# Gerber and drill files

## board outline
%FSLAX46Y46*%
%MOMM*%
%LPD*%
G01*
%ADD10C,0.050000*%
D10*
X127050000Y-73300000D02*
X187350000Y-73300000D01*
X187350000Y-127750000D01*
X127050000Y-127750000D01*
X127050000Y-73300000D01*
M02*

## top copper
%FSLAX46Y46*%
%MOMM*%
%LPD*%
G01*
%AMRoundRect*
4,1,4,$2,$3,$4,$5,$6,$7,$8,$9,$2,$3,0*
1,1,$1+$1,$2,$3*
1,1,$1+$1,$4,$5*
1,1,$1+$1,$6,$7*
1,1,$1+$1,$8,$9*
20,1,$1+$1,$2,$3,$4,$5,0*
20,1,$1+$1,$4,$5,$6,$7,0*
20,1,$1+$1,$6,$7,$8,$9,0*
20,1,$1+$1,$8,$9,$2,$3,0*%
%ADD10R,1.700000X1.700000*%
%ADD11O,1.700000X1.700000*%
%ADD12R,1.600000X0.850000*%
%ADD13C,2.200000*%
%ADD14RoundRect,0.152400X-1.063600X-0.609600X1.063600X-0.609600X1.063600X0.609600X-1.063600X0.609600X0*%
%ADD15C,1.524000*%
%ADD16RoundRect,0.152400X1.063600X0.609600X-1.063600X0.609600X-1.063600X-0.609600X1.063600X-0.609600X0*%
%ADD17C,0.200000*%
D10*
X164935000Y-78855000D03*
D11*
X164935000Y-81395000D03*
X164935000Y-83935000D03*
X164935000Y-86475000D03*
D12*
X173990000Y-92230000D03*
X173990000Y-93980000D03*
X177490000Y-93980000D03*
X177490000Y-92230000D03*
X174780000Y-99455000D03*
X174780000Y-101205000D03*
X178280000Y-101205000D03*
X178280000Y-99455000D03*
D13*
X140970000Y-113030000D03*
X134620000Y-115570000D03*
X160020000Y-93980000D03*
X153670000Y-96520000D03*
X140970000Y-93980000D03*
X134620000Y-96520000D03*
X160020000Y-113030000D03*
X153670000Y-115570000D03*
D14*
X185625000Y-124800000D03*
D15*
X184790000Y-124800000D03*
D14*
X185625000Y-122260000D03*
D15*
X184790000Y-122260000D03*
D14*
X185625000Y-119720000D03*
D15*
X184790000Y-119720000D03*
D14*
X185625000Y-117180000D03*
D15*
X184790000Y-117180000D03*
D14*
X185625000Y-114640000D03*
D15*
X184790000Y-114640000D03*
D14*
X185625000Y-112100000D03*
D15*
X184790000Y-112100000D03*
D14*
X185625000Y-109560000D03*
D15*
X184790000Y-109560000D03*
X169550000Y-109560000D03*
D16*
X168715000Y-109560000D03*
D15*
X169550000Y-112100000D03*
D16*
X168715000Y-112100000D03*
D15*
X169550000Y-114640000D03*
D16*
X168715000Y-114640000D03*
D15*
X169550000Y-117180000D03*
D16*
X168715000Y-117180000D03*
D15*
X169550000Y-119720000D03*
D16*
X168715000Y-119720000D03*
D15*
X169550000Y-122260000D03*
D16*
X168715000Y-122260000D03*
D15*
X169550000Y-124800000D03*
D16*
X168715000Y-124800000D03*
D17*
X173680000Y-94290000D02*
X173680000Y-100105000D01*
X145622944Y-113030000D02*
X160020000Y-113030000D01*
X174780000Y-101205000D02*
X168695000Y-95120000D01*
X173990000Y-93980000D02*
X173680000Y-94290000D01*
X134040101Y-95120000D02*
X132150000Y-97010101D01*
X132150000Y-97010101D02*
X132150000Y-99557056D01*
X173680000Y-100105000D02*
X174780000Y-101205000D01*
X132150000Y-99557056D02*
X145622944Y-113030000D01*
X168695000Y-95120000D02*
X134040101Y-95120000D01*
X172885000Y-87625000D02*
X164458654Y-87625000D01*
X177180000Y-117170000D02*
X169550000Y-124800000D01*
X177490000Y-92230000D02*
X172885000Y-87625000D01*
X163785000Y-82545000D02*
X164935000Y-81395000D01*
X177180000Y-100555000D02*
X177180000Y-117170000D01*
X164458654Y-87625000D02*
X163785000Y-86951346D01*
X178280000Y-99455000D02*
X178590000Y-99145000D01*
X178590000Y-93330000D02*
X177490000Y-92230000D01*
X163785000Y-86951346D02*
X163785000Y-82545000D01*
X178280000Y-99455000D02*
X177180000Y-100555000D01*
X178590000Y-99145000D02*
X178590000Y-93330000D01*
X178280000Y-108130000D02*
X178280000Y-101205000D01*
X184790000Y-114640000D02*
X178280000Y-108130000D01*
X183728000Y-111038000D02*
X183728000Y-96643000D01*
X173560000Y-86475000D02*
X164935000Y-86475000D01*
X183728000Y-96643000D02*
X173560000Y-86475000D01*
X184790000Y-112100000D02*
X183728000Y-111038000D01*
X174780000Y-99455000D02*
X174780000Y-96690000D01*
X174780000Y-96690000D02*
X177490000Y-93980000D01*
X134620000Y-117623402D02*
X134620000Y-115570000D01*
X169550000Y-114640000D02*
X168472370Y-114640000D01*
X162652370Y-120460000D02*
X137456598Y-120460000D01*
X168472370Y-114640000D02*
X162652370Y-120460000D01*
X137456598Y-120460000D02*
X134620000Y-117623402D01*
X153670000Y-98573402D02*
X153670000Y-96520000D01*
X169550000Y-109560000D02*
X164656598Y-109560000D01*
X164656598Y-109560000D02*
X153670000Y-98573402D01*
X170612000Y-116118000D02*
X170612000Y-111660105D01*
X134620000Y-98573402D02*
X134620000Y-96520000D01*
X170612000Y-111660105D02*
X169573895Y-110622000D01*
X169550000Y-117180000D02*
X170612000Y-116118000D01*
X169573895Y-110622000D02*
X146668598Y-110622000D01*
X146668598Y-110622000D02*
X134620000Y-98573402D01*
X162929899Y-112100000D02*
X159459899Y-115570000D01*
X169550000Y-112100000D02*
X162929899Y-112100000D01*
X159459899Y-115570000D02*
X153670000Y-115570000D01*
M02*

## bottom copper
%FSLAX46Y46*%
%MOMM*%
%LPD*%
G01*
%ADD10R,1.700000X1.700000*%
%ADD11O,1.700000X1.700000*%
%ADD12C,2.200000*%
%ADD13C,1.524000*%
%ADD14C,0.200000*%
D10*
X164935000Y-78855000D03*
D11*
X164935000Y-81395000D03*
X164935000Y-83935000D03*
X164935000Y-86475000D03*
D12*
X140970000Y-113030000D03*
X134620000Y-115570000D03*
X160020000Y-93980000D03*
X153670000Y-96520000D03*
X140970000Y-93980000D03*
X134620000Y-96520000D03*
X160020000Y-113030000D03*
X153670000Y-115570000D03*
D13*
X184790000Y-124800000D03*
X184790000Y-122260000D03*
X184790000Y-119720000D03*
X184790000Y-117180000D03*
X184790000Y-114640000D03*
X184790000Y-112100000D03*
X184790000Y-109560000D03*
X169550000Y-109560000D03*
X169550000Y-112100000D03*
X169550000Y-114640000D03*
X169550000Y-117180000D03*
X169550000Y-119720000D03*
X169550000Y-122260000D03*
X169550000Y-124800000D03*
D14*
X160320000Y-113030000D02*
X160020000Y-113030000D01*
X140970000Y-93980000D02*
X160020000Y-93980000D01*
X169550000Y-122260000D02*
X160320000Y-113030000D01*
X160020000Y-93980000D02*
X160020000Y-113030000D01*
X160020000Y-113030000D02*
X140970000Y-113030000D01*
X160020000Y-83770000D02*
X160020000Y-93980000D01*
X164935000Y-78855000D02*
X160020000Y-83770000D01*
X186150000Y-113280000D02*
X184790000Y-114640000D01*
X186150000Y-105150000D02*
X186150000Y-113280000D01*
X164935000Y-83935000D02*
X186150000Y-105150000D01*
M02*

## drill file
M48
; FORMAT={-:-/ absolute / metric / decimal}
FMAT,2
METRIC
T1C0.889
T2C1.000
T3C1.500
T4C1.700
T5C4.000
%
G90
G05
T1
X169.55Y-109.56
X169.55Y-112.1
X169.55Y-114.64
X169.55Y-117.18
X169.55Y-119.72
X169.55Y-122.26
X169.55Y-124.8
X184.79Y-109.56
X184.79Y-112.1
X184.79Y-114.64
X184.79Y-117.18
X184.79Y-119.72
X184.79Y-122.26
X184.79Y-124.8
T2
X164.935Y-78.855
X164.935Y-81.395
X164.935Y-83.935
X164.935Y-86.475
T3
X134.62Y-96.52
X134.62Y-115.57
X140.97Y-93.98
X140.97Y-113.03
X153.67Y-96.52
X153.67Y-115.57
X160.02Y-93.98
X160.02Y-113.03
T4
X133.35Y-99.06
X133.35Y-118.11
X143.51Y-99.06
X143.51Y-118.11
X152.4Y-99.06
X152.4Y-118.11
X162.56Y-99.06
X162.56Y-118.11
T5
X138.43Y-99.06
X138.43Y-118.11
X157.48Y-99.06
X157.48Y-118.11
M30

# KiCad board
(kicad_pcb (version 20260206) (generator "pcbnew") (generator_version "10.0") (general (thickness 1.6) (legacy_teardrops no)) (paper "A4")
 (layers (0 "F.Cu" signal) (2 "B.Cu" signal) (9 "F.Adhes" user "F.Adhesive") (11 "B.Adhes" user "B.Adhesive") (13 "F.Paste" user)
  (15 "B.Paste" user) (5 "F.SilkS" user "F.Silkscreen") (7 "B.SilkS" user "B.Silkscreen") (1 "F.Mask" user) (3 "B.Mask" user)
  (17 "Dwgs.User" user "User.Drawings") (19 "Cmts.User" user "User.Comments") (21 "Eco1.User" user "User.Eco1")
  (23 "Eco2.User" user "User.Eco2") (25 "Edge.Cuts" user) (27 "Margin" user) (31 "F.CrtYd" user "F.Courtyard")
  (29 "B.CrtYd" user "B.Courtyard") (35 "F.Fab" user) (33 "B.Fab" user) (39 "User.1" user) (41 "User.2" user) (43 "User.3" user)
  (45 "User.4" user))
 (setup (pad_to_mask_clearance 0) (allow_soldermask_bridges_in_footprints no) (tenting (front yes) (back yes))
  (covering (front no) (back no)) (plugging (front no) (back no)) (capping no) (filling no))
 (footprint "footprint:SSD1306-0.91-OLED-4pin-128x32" (layer "F.Cu") (at 128.435 76.665)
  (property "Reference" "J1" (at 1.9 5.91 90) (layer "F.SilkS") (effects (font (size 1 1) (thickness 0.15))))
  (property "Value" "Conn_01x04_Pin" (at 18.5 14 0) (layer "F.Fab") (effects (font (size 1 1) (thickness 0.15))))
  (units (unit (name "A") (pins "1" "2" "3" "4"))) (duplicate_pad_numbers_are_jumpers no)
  (pad "1" thru_hole rect (at 36.5 2.19) (size 1.7 1.7) (drill 1) (layers "*.Cu" "*.Mask") (remove_unused_layers no) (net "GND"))
  (pad "2" thru_hole oval (at 36.5 4.73) (size 1.7 1.7) (drill 1) (layers "*.Cu" "*.Mask") (remove_unused_layers no) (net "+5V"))
  (pad "3" thru_hole oval (at 36.5 7.27) (size 1.7 1.7) (drill 1) (layers "*.Cu" "*.Mask") (remove_unused_layers no) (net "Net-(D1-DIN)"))
  (pad "4" thru_hole oval (at 36.5 9.81) (size 1.7 1.7) (drill 1) (layers "*.Cu" "*.Mask") (remove_unused_layers no) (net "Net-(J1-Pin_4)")))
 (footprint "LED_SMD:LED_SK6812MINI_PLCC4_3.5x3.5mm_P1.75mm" (layer "F.Cu") (at 175.74 93.105)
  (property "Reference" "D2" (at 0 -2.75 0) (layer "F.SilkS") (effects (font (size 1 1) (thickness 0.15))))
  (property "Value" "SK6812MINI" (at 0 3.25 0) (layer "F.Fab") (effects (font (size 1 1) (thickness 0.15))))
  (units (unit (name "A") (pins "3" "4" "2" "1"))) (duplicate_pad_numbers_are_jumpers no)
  (pad "1" smd rect (at -1.75 -0.875) (size 1.6 0.85) (layers "F.Cu" "F.Mask" "F.Paste") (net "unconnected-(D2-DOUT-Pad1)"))
  (pad "2" smd rect (at -1.75 0.875) (size 1.6 0.85) (layers "F.Cu" "F.Mask" "F.Paste") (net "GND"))
  (pad "3" smd rect (at 1.75 0.875) (size 1.6 0.85) (layers "F.Cu" "F.Mask" "F.Paste") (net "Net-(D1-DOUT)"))
  (pad "4" smd rect (at 1.75 -0.875) (size 1.6 0.85) (layers "F.Cu" "F.Mask" "F.Paste") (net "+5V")))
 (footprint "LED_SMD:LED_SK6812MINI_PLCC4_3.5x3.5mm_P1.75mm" (layer "F.Cu") (at 176.53 100.33)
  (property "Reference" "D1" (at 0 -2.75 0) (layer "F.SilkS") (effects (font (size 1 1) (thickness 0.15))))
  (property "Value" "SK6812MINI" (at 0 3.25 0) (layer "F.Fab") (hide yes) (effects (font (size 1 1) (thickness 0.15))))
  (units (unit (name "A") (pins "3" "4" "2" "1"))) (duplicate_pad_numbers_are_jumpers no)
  (pad "1" smd rect (at -1.75 -0.875) (size 1.6 0.85) (layers "F.Cu" "F.Mask" "F.Paste") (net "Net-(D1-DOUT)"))
  (pad "2" smd rect (at -1.75 0.875) (size 1.6 0.85) (layers "F.Cu" "F.Mask" "F.Paste") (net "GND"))
  (pad "3" smd rect (at 1.75 0.875) (size 1.6 0.85) (layers "F.Cu" "F.Mask" "F.Paste") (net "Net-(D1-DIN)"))
  (pad "4" smd rect (at 1.75 -0.875) (size 1.6 0.85) (layers "F.Cu" "F.Mask" "F.Paste") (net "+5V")))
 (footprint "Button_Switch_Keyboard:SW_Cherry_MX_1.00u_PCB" (layer "F.Cu") (at 140.97 113.03)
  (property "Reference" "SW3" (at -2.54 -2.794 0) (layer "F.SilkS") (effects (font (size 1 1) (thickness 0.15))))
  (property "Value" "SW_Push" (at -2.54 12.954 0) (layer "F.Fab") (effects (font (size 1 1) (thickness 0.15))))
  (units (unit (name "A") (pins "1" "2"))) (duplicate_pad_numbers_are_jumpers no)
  (pad "" np_thru_hole circle (at -7.62 5.08) (size 1.7 1.7) (drill 1.7) (layers "*.Cu" "*.Mask"))
  (pad "" np_thru_hole circle (at -2.54 5.08) (size 4 4) (drill 4) (layers "*.Cu" "*.Mask"))
  (pad "" np_thru_hole circle (at 2.54 5.08) (size 1.7 1.7) (drill 1.7) (layers "*.Cu" "*.Mask"))
  (pad "1" thru_hole circle (at 0 0) (size 2.2 2.2) (drill 1.5) (layers "*.Cu" "*.Mask") (remove_unused_layers no) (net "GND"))
  (pad "2" thru_hole circle (at -6.35 2.54) (size 2.2 2.2) (drill 1.5) (layers "*.Cu" "*.Mask") (remove_unused_layers no)
   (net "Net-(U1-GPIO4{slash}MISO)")))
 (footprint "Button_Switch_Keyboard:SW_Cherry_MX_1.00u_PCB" (layer "F.Cu") (at 160.02 93.98)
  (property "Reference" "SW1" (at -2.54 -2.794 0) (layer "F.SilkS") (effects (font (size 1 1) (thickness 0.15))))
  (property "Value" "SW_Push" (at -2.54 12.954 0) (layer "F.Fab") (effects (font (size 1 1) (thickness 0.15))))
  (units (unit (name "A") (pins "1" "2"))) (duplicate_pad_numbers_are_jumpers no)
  (pad "" np_thru_hole circle (at -7.62 5.08) (size 1.7 1.7) (drill 1.7) (layers "*.Cu" "*.Mask"))
  (pad "" np_thru_hole circle (at -2.54 5.08) (size 4 4) (drill 4) (layers "*.Cu" "*.Mask"))
  (pad "" np_thru_hole circle (at 2.54 5.08) (size 1.7 1.7) (drill 1.7) (layers "*.Cu" "*.Mask"))
  (pad "1" thru_hole circle (at 0 0) (size 2.2 2.2) (drill 1.5) (layers "*.Cu" "*.Mask") (remove_unused_layers no) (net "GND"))
  (pad "2" thru_hole circle (at -6.35 2.54) (size 2.2 2.2) (drill 1.5) (layers "*.Cu" "*.Mask") (remove_unused_layers no)
   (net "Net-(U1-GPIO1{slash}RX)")))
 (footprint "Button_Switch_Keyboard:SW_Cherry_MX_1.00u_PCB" (layer "F.Cu") (at 140.97 93.98)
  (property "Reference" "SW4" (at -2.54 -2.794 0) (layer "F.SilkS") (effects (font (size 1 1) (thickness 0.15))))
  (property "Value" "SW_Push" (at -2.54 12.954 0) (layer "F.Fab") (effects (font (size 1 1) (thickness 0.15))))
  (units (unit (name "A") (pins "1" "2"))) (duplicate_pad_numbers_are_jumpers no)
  (pad "" np_thru_hole circle (at -7.62 5.08) (size 1.7 1.7) (drill 1.7) (layers "*.Cu" "*.Mask"))
  (pad "" np_thru_hole circle (at -2.54 5.08) (size 4 4) (drill 4) (layers "*.Cu" "*.Mask"))
  (pad "" np_thru_hole circle (at 2.54 5.08) (size 1.7 1.7) (drill 1.7) (layers "*.Cu" "*.Mask"))
  (pad "1" thru_hole circle (at 0 0) (size 2.2 2.2) (drill 1.5) (layers "*.Cu" "*.Mask") (remove_unused_layers no) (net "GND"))
  (pad "2" thru_hole circle (at -6.35 2.54) (size 2.2 2.2) (drill 1.5) (layers "*.Cu" "*.Mask") (remove_unused_layers no)
   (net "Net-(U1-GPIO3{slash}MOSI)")))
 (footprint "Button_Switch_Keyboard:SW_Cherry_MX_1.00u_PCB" (layer "F.Cu") (at 160.02 113.03)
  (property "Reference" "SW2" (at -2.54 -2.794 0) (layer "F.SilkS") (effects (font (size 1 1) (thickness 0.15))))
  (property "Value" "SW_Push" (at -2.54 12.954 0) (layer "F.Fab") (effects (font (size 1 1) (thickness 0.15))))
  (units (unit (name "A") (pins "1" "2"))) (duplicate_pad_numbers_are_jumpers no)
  (pad "" np_thru_hole circle (at -7.62 5.08) (size 1.7 1.7) (drill 1.7) (layers "*.Cu" "*.Mask"))
  (pad "" np_thru_hole circle (at -2.54 5.08) (size 4 4) (drill 4) (layers "*.Cu" "*.Mask"))
  (pad "" np_thru_hole circle (at 2.54 5.08) (size 1.7 1.7) (drill 1.7) (layers "*.Cu" "*.Mask"))
  (pad "1" thru_hole circle (at 0 0) (size 2.2 2.2) (drill 1.5) (layers "*.Cu" "*.Mask") (remove_unused_layers no) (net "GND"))
  (pad "2" thru_hole circle (at -6.35 2.54) (size 2.2 2.2) (drill 1.5) (layers "*.Cu" "*.Mask") (remove_unused_layers no)
   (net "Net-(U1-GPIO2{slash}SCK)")))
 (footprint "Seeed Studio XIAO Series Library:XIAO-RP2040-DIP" (layer "F.Cu") (at 177.17 117.18 -90)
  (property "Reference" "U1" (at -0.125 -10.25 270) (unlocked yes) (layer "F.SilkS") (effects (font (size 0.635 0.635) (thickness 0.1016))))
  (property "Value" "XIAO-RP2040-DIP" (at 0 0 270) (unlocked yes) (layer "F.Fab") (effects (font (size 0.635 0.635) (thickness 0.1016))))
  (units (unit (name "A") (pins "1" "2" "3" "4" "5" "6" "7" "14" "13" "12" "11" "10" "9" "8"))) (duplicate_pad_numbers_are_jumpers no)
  (pad "1" smd roundrect (at 7.62 -8.455) (size 2.432 1.524) (layers "F.Cu" "F.Mask") (roundrect_rratio 0.1)
   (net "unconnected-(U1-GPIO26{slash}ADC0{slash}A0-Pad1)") (thermal_bridge_angle 45))
  (pad "1" thru_hole circle (at 7.62 -7.62) (size 1.524 1.524) (drill 0.889) (layers "*.Cu" "*.Mask") (remove_unused_layers no)
   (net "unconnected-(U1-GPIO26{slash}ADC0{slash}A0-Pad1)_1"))
  (pad "2" smd roundrect (at 5.08 -8.455) (size 2.432 1.524) (layers "F.Cu" "F.Mask") (roundrect_rratio 0.1)
   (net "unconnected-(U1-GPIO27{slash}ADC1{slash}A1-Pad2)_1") (thermal_bridge_angle 45))
  (pad "2" thru_hole circle (at 5.08 -7.62) (size 1.524 1.524) (drill 0.889) (layers "*.Cu" "*.Mask") (remove_unused_layers no)
   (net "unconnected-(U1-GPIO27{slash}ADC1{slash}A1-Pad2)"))
  (pad "3" smd roundrect (at 2.54 -8.455) (size 2.432 1.524) (layers "F.Cu" "F.Mask") (roundrect_rratio 0.1)
   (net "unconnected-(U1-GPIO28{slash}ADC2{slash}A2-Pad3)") (thermal_bridge_angle 45))
  (pad "3" thru_hole circle (at 2.54 -7.62) (size 1.524 1.524) (drill 0.889) (layers "*.Cu" "*.Mask") (remove_unused_layers no)
   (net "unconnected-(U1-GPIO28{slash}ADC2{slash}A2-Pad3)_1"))
  (pad "4" smd roundrect (at 0 -8.455) (size 2.432 1.524) (layers "F.Cu" "F.Mask") (roundrect_rratio 0.1)
   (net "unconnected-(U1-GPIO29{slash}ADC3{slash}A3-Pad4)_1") (thermal_bridge_angle 45))
  (pad "4" thru_hole circle (at 0 -7.62) (size 1.524 1.524) (drill 0.889) (layers "*.Cu" "*.Mask") (remove_unused_layers no)
   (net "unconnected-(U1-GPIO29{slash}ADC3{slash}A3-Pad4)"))
  (pad "5" smd roundrect (at -2.54 -8.455) (size 2.432 1.524) (layers "F.Cu" "F.Mask") (roundrect_rratio 0.1) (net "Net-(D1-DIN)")
   (thermal_bridge_angle 45))
  (pad "5" thru_hole circle (at -2.54 -7.62) (size 1.524 1.524) (drill 0.889) (layers "*.Cu" "*.Mask") (remove_unused_layers no)
   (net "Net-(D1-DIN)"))
  (pad "6" smd roundrect (at -5.08 -8.455) (size 2.432 1.524) (layers "F.Cu" "F.Mask") (roundrect_rratio 0.1) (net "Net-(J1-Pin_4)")
   (thermal_bridge_angle 45))
  (pad "6" thru_hole circle (at -5.08 -7.62) (size 1.524 1.524) (drill 0.889) (layers "*.Cu" "*.Mask") (remove_unused_layers no)
   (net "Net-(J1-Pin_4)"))
  (pad "7" smd roundrect (at -7.62 -8.455) (size 2.432 1.524) (layers "F.Cu" "F.Mask") (roundrect_rratio 0.1)
   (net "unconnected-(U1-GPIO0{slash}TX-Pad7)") (thermal_bridge_angle 45))
  (pad "7" thru_hole circle (at -7.62 -7.62) (size 1.524 1.524) (drill 0.889) (layers "*.Cu" "*.Mask") (remove_unused_layers no)
   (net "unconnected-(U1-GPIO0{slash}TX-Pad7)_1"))
  (pad "8" thru_hole circle (at -7.62 7.62 180) (size 1.524 1.524) (drill 0.889) (layers "*.Cu" "*.Mask") (remove_unused_layers no)
   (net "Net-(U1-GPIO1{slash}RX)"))
  (pad "8" smd roundrect (at -7.62 8.455 180) (size 2.432 1.524) (layers "F.Cu" "F.Mask") (roundrect_rratio 0.1)
   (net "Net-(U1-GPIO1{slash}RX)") (thermal_bridge_angle 45))
  (pad "9" thru_hole circle (at -5.08 7.62 180) (size 1.524 1.524) (drill 0.889) (layers "*.Cu" "*.Mask") (remove_unused_layers no)
   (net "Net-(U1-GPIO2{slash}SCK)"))
  (pad "9" smd roundrect (at -5.08 8.455 180) (size 2.432 1.524) (layers "F.Cu" "F.Mask") (roundrect_rratio 0.1)
   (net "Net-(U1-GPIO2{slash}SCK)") (thermal_bridge_angle 45))
  (pad "10" thru_hole circle (at -2.54 7.62 180) (size 1.524 1.524) (drill 0.889) (layers "*.Cu" "*.Mask") (remove_unused_layers no)
   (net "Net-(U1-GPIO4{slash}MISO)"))
  (pad "10" smd roundrect (at -2.54 8.455 180) (size 2.432 1.524) (layers "F.Cu" "F.Mask") (roundrect_rratio 0.1)
   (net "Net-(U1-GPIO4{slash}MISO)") (thermal_bridge_angle 45))
  (pad "11" thru_hole circle (at 0 7.62 180) (size 1.524 1.524) (drill 0.889) (layers "*.Cu" "*.Mask") (remove_unused_layers no)
   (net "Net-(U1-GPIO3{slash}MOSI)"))
  (pad "11" smd roundrect (at 0 8.455 180) (size 2.432 1.524) (layers "F.Cu" "F.Mask") (roundrect_rratio 0.1)
   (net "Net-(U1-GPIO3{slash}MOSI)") (thermal_bridge_angle 45))
  (pad "12" thru_hole circle (at 2.54 7.62 180) (size 1.524 1.524) (drill 0.889) (layers "*.Cu" "*.Mask") (remove_unused_layers no)
   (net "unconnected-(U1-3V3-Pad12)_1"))
  (pad "12" smd roundrect (at 2.54 8.455 180) (size 2.432 1.524) (layers "F.Cu" "F.Mask") (roundrect_rratio 0.1)
   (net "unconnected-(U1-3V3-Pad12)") (thermal_bridge_angle 45))
  (pad "13" thru_hole circle (at 5.08 7.62 180) (size 1.524 1.524) (drill 0.889) (layers "*.Cu" "*.Mask") (remove_unused_layers no)
   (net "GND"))
  (pad "13" smd roundrect (at 5.08 8.455 180) (size 2.432 1.524) (layers "F.Cu" "F.Mask") (roundrect_rratio 0.1) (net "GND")
   (thermal_bridge_angle 45))
  (pad "14" thru_hole circle (at 7.62 7.62 180) (size 1.524 1.524) (drill 0.889) (layers "*.Cu" "*.Mask") (remove_unused_layers no)
   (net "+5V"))
  (pad "14" smd roundrect (at 7.62 8.455 180) (size 2.432 1.524) (layers "F.Cu" "F.Mask") (roundrect_rratio 0.1) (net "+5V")
   (thermal_bridge_angle 45)))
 (gr_rect (start 127.05 73.3) (end 187.35 127.75) (stroke (width 0.05) (type default)) (fill no) (layer "Edge.Cuts"))
 (segment (start 173.68 94.29) (end 173.68 100.105) (width 0.2) (layer "F.Cu") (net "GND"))
 (segment (start 145.622944 113.03) (end 160.02 113.03) (width 0.2) (layer "F.Cu") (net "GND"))
 (segment (start 174.78 101.205) (end 168.695 95.12) (width 0.2) (layer "F.Cu") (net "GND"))
 (segment (start 173.99 93.98) (end 173.68 94.29) (width 0.2) (layer "F.Cu") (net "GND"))
 (segment (start 134.040101 95.12) (end 132.15 97.010101) (width 0.2) (layer "F.Cu") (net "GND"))
 (segment (start 132.15 97.010101) (end 132.15 99.557056) (width 0.2) (layer "F.Cu") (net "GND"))
 (segment (start 173.68 100.105) (end 174.78 101.205) (width 0.2) (layer "F.Cu") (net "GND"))
 (segment (start 132.15 99.557056) (end 145.622944 113.03) (width 0.2) (layer "F.Cu") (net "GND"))
 (segment (start 168.695 95.12) (end 134.040101 95.12) (width 0.2) (layer "F.Cu") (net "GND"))
 (segment (start 160.32 113.03) (end 160.02 113.03) (width 0.2) (layer "B.Cu") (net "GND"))
 (segment (start 140.97 93.98) (end 160.02 93.98) (width 0.2) (layer "B.Cu") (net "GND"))
 (segment (start 169.55 122.26) (end 160.32 113.03) (width 0.2) (layer "B.Cu") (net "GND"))
 (segment (start 160.02 93.98) (end 160.02 113.03) (width 0.2) (layer "B.Cu") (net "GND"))
 (segment (start 160.02 113.03) (end 140.97 113.03) (width 0.2) (layer "B.Cu") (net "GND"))
 (segment (start 160.02 83.77) (end 160.02 93.98) (width 0.2) (layer "B.Cu") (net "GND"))
 (segment (start 164.935 78.855) (end 160.02 83.77) (width 0.2) (layer "B.Cu") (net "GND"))
 (segment (start 172.885 87.625) (end 164.458654 87.625) (width 0.2) (layer "F.Cu") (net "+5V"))
 (segment (start 177.18 117.17) (end 169.55 124.8) (width 0.2) (layer "F.Cu") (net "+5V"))
 (segment (start 177.49 92.23) (end 172.885 87.625) (width 0.2) (layer "F.Cu") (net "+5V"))
 (segment (start 163.785 82.545) (end 164.935 81.395) (width 0.2) (layer "F.Cu") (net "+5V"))
 (segment (start 177.18 100.555) (end 177.18 117.17) (width 0.2) (layer "F.Cu") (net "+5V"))
 (segment (start 164.458654 87.625) (end 163.785 86.951346) (width 0.2) (layer "F.Cu") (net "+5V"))
 (segment (start 178.28 99.455) (end 178.59 99.145) (width 0.2) (layer "F.Cu") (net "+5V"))
 (segment (start 178.59 93.33) (end 177.49 92.23) (width 0.2) (layer "F.Cu") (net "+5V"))
 (segment (start 163.785 86.951346) (end 163.785 82.545) (width 0.2) (layer "F.Cu") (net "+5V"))
 (segment (start 178.28 99.455) (end 177.18 100.555) (width 0.2) (layer "F.Cu") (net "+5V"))
 (segment (start 178.59 99.145) (end 178.59 93.33) (width 0.2) (layer "F.Cu") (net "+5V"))
 (segment (start 178.28 108.13) (end 178.28 101.205) (width 0.2) (layer "F.Cu") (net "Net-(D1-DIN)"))
 (segment (start 184.79 114.64) (end 178.28 108.13) (width 0.2) (layer "F.Cu") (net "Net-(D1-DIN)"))
 (segment (start 186.15 113.28) (end 184.79 114.64) (width 0.2) (layer "B.Cu") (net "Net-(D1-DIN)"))
 (segment (start 186.15 105.15) (end 186.15 113.28) (width 0.2) (layer "B.Cu") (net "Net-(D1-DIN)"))
 (segment (start 164.935 83.935) (end 186.15 105.15) (width 0.2) (layer "B.Cu") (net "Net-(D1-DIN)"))
 (segment (start 183.728 111.038) (end 183.728 96.643) (width 0.2) (layer "F.Cu") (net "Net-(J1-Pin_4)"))
 (segment (start 173.56 86.475) (end 164.935 86.475) (width 0.2) (layer "F.Cu") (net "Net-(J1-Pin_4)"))
 (segment (start 183.728 96.643) (end 173.56 86.475) (width 0.2) (layer "F.Cu") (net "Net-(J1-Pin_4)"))
 (segment (start 184.79 112.1) (end 183.728 111.038) (width 0.2) (layer "F.Cu") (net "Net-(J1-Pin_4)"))
 (segment (start 174.78 99.455) (end 174.78 96.69) (width 0.2) (layer "F.Cu") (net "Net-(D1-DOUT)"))
 (segment (start 174.78 96.69) (end 177.49 93.98) (width 0.2) (layer "F.Cu") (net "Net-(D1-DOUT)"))
 (segment (start 134.62 117.623402) (end 134.62 115.57) (width 0.2) (layer "F.Cu") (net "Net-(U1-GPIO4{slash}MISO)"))
 (segment (start 169.55 114.64) (end 168.47237 114.64) (width 0.2) (layer "F.Cu") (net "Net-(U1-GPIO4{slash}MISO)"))
 (segment (start 162.65237 120.46) (end 137.456598 120.46) (width 0.2) (layer "F.Cu") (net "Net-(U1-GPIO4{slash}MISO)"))
 (segment (start 168.47237 114.64) (end 162.65237 120.46) (width 0.2) (layer "F.Cu") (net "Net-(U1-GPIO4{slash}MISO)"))
 (segment (start 137.456598 120.46) (end 134.62 117.623402) (width 0.2) (layer "F.Cu") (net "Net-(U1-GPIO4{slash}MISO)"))
 (segment (start 153.67 98.573402) (end 153.67 96.52) (width 0.2) (layer "F.Cu") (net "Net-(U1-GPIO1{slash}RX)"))
 (segment (start 169.55 109.56) (end 164.656598 109.56) (width 0.2) (layer "F.Cu") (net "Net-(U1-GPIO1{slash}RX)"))
 (segment (start 164.656598 109.56) (end 153.67 98.573402) (width 0.2) (layer "F.Cu") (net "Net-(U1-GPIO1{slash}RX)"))
 (segment (start 170.612 116.118) (end 170.612 111.660105) (width 0.2) (layer "F.Cu") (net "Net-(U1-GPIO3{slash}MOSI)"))
 (segment (start 134.62 98.573402) (end 134.62 96.52) (width 0.2) (layer "F.Cu") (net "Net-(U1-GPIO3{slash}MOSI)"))
 (segment (start 170.612 111.660105) (end 169.573895 110.622) (width 0.2) (layer "F.Cu") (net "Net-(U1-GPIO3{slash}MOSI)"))
 (segment (start 169.55 117.18) (end 170.612 116.118) (width 0.2) (layer "F.Cu") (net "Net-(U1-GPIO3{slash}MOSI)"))
 (segment (start 169.573895 110.622) (end 146.668598 110.622) (width 0.2) (layer "F.Cu") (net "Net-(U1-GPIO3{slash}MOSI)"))
 (segment (start 146.668598 110.622) (end 134.62 98.573402) (width 0.2) (layer "F.Cu") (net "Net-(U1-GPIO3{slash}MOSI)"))
 (segment (start 162.929899 112.1) (end 159.459899 115.57) (width 0.2) (layer "F.Cu") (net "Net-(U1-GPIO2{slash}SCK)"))
 (segment (start 169.55 112.1) (end 162.929899 112.1) (width 0.2) (layer "F.Cu") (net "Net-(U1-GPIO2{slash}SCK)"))
 (segment (start 159.459899 115.57) (end 153.67 115.57) (width 0.2) (layer "F.Cu") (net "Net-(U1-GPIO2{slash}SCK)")))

